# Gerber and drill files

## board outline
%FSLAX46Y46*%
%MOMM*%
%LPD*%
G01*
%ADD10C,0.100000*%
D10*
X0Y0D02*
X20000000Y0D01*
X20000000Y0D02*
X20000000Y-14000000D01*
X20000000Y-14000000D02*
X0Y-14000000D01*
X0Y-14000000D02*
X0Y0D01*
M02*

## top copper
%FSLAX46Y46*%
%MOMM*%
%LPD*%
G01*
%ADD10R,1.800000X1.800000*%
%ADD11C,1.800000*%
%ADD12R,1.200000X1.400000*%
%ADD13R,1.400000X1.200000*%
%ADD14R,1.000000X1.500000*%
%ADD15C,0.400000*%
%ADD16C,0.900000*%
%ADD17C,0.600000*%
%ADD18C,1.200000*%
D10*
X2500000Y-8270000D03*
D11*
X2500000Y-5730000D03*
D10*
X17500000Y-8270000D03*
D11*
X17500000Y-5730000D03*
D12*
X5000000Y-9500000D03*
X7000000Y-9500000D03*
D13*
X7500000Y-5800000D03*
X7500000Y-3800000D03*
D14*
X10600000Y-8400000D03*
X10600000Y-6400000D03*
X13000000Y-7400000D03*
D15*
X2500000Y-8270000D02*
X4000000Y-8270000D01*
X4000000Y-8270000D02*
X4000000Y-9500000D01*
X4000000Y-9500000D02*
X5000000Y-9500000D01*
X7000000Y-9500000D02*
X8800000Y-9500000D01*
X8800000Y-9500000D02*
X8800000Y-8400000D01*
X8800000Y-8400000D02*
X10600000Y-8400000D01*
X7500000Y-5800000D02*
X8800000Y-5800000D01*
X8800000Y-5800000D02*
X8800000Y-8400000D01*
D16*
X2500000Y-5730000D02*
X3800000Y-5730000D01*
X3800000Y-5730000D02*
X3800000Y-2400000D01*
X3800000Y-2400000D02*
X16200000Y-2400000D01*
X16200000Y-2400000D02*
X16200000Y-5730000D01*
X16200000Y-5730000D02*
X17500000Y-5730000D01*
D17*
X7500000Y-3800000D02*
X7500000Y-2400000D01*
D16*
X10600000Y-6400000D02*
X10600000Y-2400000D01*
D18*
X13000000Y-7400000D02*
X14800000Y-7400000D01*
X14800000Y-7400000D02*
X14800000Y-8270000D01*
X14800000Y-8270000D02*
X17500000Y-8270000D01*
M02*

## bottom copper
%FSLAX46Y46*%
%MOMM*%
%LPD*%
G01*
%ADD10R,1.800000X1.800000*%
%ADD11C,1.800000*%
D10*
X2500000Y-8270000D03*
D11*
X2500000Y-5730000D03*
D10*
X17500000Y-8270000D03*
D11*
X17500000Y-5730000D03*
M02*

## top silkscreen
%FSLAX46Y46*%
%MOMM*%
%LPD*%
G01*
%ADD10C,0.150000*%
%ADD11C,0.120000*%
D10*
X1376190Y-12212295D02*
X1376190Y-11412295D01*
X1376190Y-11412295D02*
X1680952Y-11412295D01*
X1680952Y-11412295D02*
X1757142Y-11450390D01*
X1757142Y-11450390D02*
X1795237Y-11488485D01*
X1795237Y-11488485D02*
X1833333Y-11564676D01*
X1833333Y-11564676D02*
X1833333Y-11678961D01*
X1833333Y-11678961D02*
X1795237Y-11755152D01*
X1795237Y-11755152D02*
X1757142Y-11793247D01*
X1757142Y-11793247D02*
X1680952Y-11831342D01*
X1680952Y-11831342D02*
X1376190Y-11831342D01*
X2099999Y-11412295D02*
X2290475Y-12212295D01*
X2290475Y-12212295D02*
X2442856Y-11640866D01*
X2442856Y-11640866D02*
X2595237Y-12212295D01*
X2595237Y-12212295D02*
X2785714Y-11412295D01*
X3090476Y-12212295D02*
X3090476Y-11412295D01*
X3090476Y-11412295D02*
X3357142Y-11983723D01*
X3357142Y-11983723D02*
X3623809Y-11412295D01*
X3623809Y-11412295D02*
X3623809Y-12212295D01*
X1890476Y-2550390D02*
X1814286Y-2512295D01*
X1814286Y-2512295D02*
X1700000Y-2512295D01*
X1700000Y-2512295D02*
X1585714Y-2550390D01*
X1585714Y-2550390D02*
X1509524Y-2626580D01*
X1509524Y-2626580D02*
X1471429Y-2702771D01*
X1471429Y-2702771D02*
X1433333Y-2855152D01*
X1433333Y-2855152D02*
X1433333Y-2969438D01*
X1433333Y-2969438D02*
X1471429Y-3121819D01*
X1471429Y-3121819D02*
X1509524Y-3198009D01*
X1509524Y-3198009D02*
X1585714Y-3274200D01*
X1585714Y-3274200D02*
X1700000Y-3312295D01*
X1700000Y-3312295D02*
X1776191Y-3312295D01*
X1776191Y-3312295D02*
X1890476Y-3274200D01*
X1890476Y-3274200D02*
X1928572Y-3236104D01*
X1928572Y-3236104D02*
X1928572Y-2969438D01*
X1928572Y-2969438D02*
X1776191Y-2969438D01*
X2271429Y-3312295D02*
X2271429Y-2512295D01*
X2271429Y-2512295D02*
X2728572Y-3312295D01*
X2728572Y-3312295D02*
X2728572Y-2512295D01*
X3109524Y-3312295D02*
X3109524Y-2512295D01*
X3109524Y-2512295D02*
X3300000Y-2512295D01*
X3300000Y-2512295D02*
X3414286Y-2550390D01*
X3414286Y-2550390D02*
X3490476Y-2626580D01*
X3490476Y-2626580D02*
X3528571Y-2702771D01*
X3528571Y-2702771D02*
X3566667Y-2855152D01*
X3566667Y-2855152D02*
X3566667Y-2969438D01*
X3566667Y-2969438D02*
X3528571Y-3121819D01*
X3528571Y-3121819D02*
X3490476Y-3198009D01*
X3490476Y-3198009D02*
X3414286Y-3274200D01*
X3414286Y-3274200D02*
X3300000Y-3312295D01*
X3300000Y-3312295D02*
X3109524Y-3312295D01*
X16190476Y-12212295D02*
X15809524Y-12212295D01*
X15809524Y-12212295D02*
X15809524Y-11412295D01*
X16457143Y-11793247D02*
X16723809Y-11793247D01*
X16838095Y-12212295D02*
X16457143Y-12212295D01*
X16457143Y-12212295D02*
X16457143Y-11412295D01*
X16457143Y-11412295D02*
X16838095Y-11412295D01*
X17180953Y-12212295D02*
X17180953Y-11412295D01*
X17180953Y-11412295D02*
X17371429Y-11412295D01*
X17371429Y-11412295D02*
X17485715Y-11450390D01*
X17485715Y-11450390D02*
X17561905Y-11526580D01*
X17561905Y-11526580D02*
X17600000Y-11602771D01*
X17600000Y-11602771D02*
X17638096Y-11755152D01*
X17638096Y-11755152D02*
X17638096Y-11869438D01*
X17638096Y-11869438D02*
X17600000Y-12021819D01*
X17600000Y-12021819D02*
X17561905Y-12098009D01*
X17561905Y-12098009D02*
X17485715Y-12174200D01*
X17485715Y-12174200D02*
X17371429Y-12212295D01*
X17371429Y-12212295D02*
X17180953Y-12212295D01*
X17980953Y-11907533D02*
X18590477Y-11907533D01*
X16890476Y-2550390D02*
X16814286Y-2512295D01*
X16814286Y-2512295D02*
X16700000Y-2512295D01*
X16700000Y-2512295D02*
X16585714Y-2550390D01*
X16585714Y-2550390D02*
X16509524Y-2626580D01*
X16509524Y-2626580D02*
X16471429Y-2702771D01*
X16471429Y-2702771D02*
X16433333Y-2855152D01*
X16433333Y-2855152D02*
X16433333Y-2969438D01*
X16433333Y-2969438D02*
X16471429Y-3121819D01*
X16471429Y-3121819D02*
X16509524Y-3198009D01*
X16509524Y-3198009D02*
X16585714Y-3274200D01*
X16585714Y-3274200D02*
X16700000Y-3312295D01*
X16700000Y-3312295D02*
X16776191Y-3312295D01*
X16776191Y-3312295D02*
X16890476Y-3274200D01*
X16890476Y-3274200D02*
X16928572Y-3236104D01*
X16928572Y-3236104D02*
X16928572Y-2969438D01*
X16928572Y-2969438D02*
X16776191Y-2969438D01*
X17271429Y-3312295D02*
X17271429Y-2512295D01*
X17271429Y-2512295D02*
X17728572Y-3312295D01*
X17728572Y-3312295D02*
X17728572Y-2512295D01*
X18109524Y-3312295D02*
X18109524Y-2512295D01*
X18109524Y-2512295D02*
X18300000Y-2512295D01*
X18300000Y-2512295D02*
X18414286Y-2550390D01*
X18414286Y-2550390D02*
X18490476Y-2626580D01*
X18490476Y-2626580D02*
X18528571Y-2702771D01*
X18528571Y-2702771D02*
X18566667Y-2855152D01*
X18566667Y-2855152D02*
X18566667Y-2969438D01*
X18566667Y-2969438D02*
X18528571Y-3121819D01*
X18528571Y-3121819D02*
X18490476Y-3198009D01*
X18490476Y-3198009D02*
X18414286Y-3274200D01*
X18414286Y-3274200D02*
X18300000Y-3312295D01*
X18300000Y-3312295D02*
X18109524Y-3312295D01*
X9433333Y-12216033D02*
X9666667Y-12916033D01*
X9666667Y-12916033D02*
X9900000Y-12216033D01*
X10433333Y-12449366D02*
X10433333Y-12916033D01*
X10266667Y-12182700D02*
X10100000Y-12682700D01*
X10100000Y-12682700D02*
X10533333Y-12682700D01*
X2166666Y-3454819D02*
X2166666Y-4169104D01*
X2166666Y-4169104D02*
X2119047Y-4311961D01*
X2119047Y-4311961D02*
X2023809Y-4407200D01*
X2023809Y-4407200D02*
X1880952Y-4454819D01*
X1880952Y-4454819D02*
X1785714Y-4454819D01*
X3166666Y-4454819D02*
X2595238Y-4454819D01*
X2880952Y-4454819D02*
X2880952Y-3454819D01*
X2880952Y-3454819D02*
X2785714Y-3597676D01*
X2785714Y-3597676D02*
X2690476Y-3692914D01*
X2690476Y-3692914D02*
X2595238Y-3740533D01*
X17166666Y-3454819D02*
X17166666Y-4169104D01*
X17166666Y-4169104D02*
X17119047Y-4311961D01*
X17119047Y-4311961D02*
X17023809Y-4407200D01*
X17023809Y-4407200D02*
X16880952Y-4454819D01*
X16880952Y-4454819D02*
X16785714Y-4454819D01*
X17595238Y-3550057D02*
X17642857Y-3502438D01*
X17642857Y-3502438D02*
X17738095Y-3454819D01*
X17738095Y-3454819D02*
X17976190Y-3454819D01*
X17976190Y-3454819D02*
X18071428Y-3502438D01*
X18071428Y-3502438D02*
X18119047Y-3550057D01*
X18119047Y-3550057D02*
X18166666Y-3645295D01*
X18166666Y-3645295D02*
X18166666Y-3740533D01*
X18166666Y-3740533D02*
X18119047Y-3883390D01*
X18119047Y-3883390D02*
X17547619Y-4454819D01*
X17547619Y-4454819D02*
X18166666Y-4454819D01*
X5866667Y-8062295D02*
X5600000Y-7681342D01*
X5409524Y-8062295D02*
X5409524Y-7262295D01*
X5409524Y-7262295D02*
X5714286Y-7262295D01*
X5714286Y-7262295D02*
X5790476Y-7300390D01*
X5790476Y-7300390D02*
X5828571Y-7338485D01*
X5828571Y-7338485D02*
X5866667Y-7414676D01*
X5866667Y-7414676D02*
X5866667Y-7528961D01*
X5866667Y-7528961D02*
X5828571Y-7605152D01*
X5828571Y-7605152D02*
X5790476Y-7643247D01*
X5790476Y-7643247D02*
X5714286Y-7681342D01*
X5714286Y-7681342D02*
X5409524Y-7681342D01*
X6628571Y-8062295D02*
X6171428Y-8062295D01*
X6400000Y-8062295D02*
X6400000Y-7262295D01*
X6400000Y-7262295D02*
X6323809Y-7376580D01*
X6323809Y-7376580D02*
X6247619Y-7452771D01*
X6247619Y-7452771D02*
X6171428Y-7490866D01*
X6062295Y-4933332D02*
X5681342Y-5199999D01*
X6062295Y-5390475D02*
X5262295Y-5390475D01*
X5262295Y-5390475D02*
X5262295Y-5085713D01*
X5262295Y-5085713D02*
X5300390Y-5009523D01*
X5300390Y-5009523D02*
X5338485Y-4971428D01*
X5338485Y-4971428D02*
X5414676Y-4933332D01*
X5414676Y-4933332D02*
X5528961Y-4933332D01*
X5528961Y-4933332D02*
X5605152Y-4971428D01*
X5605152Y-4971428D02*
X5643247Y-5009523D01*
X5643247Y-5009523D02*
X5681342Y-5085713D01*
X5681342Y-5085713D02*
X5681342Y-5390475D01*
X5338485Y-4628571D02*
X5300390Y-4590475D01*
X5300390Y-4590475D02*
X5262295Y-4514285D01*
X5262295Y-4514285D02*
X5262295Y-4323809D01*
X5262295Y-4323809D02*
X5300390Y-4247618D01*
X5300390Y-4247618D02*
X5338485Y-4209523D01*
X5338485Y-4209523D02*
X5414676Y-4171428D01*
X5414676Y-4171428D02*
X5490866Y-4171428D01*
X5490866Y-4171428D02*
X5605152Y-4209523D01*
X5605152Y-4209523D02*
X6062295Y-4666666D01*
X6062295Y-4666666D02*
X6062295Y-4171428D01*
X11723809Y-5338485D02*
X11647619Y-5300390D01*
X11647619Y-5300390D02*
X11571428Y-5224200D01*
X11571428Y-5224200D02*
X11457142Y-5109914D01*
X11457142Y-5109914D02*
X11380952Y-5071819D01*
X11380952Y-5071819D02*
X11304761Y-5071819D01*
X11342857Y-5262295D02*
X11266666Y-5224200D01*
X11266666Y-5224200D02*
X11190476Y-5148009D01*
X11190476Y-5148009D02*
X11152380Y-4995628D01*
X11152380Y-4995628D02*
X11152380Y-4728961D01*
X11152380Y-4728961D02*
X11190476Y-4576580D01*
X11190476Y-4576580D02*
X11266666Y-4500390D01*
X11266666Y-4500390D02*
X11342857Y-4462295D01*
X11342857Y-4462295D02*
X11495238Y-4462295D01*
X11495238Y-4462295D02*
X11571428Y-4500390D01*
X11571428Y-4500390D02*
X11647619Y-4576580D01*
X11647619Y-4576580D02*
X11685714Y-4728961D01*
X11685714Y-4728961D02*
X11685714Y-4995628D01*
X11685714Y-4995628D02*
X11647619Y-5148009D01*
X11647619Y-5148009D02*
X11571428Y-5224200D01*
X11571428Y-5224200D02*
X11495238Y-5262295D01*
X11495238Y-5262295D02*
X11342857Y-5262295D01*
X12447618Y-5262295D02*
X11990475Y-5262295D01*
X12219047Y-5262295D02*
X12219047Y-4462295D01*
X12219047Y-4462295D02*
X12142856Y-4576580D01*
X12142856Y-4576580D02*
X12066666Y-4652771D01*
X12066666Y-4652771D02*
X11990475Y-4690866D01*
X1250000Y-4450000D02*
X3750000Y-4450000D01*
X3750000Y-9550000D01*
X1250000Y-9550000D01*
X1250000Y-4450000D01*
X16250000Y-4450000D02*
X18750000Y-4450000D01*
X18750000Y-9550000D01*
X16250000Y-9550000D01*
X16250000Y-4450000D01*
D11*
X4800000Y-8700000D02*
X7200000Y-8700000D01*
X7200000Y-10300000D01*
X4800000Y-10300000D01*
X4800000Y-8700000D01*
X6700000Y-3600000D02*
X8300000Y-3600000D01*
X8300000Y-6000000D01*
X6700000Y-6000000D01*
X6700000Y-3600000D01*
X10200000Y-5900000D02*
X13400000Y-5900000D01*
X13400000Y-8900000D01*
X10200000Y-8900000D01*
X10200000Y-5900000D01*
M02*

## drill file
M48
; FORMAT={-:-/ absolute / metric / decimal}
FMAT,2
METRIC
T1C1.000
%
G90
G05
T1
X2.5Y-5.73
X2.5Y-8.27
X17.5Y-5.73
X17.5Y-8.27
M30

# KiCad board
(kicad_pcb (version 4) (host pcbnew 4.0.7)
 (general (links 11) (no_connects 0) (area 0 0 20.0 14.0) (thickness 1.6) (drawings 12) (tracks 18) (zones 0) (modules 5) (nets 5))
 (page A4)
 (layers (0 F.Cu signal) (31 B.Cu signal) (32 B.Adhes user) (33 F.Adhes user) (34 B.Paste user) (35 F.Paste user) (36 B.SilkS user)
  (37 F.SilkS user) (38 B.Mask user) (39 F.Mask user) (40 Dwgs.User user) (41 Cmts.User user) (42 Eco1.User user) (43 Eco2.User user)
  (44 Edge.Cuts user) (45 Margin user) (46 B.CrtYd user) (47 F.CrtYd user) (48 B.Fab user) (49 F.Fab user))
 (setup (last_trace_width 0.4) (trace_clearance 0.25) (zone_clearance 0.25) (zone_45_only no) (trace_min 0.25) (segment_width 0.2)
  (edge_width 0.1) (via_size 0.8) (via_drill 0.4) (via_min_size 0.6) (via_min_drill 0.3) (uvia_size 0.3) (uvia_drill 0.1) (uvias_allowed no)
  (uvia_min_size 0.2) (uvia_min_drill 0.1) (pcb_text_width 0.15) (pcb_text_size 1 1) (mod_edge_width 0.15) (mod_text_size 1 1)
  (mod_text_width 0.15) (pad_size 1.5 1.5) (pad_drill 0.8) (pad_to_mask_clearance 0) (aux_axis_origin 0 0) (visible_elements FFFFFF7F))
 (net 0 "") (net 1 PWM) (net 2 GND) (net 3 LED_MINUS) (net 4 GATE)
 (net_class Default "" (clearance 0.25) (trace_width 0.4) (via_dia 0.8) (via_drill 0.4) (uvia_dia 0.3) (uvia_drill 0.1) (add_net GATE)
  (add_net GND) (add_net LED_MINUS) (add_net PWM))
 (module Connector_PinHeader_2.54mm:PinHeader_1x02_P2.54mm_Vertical (layer F.Cu) (at 2.5 7)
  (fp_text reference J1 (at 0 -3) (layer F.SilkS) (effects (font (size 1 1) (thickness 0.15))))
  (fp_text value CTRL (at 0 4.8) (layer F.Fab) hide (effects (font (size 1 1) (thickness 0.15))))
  (fp_rect (start -1.25 -2.55) (end 1.25 2.55) (layer F.SilkS) (width 0.15))
  (pad 1 thru_hole rect (at 0 1.27) (size 1.8 1.8) (drill 1) (layers *.Cu *.Mask) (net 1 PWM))
  (pad 2 thru_hole circle (at 0 -1.27) (size 1.8 1.8) (drill 1) (layers *.Cu *.Mask) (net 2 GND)))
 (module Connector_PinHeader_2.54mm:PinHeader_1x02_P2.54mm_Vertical (layer F.Cu) (at 17.5 7)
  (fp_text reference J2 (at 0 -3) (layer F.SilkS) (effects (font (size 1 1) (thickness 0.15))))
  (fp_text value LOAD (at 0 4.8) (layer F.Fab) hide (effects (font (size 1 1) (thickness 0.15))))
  (fp_rect (start -1.25 -2.55) (end 1.25 2.55) (layer F.SilkS) (width 0.15))
  (pad 1 thru_hole rect (at 0 1.27) (size 1.8 1.8) (drill 1) (layers *.Cu *.Mask) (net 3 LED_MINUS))
  (pad 2 thru_hole circle (at 0 -1.27) (size 1.8 1.8) (drill 1) (layers *.Cu *.Mask) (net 2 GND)))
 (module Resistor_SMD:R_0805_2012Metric (layer F.Cu) (at 6 9.5)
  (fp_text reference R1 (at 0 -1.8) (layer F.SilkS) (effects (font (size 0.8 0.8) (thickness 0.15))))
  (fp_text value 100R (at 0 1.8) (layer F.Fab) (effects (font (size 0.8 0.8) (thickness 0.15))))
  (fp_rect (start -1.2 -0.8) (end 1.2 0.8) (layer F.SilkS) (width 0.12))
  (pad 1 smd rect (at -1 0) (size 1.2 1.4) (layers F.Cu F.Paste F.Mask) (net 1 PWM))
  (pad 2 smd rect (at 1 0) (size 1.2 1.4) (layers F.Cu F.Paste F.Mask) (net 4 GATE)))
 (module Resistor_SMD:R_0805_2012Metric (layer F.Cu) (at 7.5 4.8 90)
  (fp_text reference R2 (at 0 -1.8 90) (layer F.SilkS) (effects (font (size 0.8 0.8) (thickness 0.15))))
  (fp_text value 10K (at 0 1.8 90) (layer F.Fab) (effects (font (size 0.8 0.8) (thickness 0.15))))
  (fp_rect (start -1.2 -0.8) (end 1.2 0.8) (layer F.SilkS) (width 0.12))
  (pad 1 smd rect (at -1 0 90) (size 1.2 1.4) (layers F.Cu F.Paste F.Mask) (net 4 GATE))
  (pad 2 smd rect (at 1 0 90) (size 1.2 1.4) (layers F.Cu F.Paste F.Mask) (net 2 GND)))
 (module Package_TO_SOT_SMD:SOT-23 (layer F.Cu) (at 11.8 7.4)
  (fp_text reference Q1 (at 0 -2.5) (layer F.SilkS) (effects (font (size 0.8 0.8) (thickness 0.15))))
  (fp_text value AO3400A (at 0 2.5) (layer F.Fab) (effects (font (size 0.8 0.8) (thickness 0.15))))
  (fp_rect (start -1.6 -1.5) (end 1.6 1.5) (layer F.SilkS) (width 0.12))
  (pad 1 smd rect (at -1.2 1) (size 1 1.5) (layers F.Cu F.Paste F.Mask) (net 4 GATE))
  (pad 2 smd rect (at -1.2 -1) (size 1 1.5) (layers F.Cu F.Paste F.Mask) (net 2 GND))
  (pad 3 smd rect (at 1.2 0) (size 1 1.5) (layers F.Cu F.Paste F.Mask) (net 3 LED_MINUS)))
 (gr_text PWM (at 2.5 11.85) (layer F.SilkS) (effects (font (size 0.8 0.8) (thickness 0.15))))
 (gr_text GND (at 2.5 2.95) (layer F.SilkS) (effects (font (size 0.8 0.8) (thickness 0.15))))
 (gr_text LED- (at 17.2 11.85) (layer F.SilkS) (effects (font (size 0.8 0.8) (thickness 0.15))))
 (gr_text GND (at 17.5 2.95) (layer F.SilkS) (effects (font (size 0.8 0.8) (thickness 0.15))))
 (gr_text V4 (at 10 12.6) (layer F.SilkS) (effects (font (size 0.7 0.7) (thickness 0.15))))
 (gr_line (start 0 0) (end 20.0 0) (layer Edge.Cuts) (width 0.1))
 (gr_line (start 20.0 0) (end 20.0 14.0) (layer Edge.Cuts) (width 0.1))
 (gr_line (start 20.0 14.0) (end 0 14.0) (layer Edge.Cuts) (width 0.1))
 (gr_line (start 0 14.0) (end 0 0) (layer Edge.Cuts) (width 0.1))
 (segment (start 2.5 8.27) (end 4.0 8.27) (width 0.4) (layer F.Cu) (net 1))
 (segment (start 4.0 8.27) (end 4.0 9.5) (width 0.4) (layer F.Cu) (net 1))
 (segment (start 4.0 9.5) (end 5.0 9.5) (width 0.4) (layer F.Cu) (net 1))
 (segment (start 7.0 9.5) (end 8.8 9.5) (width 0.4) (layer F.Cu) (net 4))
 (segment (start 8.8 9.5) (end 8.8 8.4) (width 0.4) (layer F.Cu) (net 4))
 (segment (start 8.8 8.4) (end 10.6 8.4) (width 0.4) (layer F.Cu) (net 4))
 (segment (start 7.5 5.8) (end 8.8 5.8) (width 0.4) (layer F.Cu) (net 4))
 (segment (start 8.8 5.8) (end 8.8 8.4) (width 0.4) (layer F.Cu) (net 4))
 (segment (start 2.5 5.73) (end 3.8 5.73) (width 0.9) (layer F.Cu) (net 2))
 (segment (start 3.8 5.73) (end 3.8 2.4) (width 0.9) (layer F.Cu) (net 2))
 (segment (start 3.8 2.4) (end 16.2 2.4) (width 0.9) (layer F.Cu) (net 2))
 (segment (start 16.2 2.4) (end 16.2 5.73) (width 0.9) (layer F.Cu) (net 2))
 (segment (start 16.2 5.73) (end 17.5 5.73) (width 0.9) (layer F.Cu) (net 2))
 (segment (start 7.5 3.8) (end 7.5 2.4) (width 0.6) (layer F.Cu) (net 2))
 (segment (start 10.6 6.4) (end 10.6 2.4) (width 0.9) (layer F.Cu) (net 2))
 (segment (start 13.0 7.4) (end 14.8 7.4) (width 1.2) (layer F.Cu) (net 3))
 (segment (start 14.8 7.4) (end 14.8 8.27) (width 1.2) (layer F.Cu) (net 3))
 (segment (start 14.8 8.27) (end 17.5 8.27) (width 1.2) (layer F.Cu) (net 3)))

